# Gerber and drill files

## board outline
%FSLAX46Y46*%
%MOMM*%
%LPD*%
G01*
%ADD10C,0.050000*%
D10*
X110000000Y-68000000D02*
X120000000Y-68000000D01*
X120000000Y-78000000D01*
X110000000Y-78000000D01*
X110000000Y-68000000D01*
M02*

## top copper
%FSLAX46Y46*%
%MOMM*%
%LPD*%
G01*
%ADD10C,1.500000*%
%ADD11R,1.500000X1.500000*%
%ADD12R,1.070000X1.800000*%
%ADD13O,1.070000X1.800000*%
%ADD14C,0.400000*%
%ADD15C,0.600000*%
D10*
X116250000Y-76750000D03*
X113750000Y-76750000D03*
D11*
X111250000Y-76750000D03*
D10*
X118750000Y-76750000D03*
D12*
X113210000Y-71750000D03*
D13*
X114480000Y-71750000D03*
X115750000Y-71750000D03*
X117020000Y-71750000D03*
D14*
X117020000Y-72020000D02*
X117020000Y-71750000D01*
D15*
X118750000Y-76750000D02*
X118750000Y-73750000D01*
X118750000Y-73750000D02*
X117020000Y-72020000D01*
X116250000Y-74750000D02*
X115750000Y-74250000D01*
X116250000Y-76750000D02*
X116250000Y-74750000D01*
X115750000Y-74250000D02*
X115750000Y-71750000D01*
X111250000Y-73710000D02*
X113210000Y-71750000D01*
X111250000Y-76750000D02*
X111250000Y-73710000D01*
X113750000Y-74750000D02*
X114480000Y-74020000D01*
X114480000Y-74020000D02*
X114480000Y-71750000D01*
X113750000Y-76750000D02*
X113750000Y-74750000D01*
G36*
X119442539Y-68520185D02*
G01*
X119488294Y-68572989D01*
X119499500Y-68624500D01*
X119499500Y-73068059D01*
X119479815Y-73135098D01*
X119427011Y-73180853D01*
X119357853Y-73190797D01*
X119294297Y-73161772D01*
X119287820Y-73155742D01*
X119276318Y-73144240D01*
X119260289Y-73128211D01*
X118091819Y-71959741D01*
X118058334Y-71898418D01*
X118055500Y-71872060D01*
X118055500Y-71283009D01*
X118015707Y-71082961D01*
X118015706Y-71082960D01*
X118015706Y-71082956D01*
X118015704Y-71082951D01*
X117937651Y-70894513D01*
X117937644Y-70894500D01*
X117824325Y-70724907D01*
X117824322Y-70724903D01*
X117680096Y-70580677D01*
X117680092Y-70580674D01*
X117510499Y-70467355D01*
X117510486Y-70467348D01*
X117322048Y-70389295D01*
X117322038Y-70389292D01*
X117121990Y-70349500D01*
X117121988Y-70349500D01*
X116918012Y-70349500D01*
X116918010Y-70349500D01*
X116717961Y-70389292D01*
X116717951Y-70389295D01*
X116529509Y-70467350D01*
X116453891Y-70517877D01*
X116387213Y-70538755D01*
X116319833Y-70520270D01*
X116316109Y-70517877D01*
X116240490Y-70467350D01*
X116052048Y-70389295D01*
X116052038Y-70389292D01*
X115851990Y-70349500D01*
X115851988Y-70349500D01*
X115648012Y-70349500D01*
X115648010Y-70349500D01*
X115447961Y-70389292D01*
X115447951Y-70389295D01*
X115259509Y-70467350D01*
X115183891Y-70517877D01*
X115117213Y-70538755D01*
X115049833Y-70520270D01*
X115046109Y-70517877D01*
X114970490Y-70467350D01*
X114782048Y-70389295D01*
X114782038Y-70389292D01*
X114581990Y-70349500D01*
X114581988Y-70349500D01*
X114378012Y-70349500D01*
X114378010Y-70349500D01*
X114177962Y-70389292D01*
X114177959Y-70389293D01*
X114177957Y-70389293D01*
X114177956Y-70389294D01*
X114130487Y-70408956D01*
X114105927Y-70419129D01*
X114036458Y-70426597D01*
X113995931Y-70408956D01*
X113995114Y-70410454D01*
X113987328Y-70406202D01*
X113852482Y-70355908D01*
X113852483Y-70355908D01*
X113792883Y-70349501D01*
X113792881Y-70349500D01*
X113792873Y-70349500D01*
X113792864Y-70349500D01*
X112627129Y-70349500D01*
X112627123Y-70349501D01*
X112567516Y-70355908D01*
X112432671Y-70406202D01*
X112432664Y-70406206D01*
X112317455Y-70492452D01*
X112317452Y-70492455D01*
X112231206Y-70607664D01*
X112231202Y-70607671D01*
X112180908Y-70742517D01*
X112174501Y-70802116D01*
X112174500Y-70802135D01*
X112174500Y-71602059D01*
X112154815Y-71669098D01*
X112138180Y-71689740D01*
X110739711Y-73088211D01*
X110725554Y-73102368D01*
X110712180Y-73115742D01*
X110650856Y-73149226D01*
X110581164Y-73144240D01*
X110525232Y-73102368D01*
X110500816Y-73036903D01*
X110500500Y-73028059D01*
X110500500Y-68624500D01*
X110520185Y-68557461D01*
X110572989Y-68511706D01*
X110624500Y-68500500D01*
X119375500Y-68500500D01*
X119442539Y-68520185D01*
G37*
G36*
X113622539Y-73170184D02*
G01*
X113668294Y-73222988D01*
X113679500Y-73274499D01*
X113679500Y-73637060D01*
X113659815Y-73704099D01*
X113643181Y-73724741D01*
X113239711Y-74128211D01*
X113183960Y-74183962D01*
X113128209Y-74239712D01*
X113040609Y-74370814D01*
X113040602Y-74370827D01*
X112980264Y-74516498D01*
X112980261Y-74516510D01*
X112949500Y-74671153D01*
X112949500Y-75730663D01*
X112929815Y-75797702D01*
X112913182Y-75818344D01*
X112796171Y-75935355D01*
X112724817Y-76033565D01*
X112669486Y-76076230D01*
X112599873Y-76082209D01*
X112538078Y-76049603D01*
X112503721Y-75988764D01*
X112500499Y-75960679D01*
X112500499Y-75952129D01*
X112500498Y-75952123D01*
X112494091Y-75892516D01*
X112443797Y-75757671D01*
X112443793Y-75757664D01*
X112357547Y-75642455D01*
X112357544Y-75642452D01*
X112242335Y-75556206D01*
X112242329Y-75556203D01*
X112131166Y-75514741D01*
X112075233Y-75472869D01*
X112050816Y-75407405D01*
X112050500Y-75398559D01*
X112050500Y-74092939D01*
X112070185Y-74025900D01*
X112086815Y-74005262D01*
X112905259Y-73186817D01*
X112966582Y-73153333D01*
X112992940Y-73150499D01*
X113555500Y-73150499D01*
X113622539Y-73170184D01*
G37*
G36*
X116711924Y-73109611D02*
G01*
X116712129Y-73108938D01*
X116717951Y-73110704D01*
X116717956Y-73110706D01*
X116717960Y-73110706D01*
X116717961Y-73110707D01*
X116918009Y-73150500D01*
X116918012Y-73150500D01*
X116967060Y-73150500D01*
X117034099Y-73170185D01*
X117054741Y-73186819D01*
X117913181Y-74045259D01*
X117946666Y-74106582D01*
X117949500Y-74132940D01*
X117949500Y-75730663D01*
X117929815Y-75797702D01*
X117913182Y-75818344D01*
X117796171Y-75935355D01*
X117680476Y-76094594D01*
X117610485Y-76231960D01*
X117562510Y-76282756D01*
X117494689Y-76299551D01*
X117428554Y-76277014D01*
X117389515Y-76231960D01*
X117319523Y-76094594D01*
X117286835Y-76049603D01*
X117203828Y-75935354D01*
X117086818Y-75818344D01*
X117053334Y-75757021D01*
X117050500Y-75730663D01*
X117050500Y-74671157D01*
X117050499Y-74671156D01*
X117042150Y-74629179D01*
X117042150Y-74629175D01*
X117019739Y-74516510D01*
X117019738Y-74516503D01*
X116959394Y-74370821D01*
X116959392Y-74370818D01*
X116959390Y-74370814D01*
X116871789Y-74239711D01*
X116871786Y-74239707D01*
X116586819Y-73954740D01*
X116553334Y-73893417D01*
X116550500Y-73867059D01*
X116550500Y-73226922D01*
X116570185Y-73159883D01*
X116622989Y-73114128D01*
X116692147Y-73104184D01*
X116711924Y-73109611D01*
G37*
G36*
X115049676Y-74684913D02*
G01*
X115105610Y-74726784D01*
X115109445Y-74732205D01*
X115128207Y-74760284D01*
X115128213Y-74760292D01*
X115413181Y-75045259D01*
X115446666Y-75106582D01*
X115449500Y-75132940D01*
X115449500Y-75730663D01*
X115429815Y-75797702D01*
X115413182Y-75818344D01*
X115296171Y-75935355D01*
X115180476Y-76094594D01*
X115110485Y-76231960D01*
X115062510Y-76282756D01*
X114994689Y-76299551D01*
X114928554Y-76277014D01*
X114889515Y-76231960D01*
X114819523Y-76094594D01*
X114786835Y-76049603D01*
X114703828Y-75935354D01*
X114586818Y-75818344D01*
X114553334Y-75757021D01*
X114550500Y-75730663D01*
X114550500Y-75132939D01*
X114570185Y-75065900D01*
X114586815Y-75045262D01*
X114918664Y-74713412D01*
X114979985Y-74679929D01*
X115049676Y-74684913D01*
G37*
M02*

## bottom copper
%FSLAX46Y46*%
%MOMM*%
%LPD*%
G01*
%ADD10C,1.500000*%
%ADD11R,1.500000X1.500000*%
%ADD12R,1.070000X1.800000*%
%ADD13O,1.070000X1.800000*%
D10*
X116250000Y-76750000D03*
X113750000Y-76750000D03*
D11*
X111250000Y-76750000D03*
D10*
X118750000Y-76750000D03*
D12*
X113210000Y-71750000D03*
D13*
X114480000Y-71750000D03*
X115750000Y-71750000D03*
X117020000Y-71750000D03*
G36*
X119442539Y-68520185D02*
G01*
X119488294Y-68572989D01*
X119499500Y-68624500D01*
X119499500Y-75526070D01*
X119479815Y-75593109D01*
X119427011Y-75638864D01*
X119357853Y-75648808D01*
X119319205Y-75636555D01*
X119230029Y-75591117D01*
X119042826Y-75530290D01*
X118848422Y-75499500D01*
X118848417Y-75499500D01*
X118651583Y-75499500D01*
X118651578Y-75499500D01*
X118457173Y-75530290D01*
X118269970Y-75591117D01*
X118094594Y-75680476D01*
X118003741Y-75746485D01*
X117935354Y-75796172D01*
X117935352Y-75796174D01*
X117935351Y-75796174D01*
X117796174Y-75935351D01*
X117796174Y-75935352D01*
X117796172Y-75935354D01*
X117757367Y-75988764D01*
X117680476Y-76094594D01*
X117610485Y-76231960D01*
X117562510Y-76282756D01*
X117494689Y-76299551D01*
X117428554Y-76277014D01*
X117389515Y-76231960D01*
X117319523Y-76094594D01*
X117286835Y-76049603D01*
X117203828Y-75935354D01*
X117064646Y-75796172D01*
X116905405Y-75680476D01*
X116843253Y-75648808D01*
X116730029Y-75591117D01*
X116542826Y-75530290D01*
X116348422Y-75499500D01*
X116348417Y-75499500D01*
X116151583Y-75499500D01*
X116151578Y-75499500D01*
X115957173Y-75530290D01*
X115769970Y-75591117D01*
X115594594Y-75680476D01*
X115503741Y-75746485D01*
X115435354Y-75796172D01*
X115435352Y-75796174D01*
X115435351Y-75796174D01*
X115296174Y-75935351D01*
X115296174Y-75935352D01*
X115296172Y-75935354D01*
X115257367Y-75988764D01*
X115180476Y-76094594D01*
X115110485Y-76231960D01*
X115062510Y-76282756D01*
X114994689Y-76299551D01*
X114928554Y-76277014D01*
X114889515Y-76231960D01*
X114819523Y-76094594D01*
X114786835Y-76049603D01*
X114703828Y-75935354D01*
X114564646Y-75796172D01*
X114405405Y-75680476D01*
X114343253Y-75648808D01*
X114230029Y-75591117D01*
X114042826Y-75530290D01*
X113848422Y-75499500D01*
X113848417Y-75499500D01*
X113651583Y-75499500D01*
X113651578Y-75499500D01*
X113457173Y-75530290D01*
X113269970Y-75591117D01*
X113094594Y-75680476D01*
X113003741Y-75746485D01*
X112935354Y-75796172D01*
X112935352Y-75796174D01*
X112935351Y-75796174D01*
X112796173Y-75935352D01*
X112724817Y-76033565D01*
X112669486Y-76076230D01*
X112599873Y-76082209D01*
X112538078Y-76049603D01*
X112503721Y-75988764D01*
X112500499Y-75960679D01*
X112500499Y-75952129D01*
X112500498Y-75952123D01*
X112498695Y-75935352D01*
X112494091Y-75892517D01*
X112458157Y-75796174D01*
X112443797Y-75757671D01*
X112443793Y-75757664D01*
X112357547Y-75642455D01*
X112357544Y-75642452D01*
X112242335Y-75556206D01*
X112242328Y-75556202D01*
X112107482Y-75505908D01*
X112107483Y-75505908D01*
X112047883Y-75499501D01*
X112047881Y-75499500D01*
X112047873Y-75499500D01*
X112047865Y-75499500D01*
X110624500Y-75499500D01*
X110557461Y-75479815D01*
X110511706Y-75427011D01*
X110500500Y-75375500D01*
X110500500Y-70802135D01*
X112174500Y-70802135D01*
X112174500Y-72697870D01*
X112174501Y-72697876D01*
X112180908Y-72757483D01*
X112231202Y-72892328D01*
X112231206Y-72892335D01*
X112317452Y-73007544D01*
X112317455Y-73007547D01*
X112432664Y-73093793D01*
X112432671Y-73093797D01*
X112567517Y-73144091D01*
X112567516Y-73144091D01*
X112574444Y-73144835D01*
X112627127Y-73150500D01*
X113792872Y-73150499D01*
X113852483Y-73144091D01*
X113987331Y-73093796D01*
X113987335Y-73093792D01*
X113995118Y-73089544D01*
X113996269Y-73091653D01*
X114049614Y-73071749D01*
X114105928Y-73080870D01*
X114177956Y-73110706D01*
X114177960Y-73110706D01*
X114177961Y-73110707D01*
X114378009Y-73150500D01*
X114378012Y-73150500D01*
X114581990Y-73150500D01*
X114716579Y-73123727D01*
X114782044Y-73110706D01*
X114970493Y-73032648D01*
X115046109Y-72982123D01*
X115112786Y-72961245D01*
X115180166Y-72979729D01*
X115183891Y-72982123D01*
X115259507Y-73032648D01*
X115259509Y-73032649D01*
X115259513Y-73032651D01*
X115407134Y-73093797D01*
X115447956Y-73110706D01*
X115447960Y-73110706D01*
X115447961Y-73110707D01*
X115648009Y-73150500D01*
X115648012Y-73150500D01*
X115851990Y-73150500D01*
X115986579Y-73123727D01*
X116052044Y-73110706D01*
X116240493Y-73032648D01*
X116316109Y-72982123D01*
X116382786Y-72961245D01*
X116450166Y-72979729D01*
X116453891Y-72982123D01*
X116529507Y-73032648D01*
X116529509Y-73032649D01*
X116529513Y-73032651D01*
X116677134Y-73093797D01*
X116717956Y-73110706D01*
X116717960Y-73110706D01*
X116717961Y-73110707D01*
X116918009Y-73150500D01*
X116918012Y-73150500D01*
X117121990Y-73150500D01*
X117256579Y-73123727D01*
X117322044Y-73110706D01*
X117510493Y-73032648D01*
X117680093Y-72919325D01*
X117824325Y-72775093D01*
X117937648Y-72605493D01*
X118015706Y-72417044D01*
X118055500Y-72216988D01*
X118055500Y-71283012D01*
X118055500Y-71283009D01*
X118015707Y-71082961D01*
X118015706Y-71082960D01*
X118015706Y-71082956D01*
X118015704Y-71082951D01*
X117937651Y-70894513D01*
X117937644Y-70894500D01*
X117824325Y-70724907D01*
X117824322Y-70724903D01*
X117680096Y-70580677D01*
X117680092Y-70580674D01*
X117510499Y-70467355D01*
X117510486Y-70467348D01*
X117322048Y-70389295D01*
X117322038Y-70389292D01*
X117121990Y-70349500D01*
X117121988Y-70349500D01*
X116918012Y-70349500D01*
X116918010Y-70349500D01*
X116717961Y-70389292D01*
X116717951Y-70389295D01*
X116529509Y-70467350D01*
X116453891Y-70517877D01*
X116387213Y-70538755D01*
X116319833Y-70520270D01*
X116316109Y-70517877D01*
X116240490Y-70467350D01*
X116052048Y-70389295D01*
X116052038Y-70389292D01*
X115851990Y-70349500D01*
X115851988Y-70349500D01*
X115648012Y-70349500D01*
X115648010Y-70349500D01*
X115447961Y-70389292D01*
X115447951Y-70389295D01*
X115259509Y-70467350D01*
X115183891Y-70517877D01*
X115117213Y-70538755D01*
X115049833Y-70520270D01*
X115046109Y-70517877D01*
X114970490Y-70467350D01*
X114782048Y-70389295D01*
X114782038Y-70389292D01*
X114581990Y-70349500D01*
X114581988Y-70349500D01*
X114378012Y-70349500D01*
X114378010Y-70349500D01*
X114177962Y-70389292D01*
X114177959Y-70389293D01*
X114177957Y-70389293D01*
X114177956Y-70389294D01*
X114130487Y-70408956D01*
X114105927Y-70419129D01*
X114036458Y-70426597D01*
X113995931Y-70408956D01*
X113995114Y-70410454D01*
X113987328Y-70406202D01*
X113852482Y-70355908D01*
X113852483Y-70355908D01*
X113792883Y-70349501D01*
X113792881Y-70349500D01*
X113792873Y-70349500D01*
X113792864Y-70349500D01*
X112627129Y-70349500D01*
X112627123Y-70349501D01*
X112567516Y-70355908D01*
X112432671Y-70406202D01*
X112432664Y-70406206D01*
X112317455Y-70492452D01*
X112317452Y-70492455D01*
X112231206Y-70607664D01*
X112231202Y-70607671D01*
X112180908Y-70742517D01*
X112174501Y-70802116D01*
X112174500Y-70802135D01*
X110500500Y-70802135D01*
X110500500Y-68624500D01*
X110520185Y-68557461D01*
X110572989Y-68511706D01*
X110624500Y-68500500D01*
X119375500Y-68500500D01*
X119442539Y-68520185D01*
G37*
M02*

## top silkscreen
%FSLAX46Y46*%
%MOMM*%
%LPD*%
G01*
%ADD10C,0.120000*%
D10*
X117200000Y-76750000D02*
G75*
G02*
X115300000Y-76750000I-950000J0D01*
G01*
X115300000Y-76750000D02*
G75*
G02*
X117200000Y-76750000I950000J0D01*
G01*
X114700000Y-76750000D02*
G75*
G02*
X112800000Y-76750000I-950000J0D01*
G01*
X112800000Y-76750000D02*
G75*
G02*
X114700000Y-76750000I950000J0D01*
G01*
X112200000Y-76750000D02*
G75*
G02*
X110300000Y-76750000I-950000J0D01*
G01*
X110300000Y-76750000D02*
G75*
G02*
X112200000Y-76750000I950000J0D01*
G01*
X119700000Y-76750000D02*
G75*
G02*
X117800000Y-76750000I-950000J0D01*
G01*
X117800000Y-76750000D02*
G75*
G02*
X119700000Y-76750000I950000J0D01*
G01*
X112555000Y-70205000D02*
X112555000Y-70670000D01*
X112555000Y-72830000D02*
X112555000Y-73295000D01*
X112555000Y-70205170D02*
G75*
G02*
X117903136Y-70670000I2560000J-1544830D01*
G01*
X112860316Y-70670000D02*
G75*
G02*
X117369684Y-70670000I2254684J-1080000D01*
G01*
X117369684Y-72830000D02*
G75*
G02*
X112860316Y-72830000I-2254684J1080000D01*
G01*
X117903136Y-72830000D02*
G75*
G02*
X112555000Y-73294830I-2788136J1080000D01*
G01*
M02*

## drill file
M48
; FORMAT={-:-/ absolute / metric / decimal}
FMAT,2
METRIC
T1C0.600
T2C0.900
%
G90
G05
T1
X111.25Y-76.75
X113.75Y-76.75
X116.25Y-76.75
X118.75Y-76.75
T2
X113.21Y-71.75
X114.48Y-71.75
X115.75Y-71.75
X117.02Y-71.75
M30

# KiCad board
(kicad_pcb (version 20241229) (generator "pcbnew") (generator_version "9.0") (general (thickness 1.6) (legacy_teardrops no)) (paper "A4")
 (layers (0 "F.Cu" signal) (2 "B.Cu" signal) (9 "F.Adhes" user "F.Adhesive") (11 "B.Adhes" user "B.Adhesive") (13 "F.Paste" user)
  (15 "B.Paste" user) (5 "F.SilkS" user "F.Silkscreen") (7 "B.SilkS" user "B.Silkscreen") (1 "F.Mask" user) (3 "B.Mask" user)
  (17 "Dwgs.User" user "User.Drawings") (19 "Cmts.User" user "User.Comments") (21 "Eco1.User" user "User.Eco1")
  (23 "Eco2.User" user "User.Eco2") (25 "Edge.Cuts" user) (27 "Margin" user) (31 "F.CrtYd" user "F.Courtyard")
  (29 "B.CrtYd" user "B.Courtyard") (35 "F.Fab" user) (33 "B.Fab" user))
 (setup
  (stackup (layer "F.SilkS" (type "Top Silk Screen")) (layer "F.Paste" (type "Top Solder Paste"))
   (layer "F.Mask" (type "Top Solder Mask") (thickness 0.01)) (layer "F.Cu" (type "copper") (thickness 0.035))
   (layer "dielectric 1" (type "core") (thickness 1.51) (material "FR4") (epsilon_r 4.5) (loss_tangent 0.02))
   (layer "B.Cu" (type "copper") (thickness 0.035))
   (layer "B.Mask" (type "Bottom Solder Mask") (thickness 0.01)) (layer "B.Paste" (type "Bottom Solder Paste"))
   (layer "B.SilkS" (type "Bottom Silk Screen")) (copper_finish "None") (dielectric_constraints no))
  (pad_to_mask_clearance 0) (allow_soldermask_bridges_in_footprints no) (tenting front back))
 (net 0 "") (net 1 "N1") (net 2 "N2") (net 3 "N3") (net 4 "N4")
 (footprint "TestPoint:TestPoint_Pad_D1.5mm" (layer "F.Cu") (at 116.25 76.75)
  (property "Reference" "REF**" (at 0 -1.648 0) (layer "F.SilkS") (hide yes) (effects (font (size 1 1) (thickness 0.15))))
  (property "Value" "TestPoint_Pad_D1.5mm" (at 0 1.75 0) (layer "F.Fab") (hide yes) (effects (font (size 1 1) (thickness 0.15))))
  (fp_circle (center 0 0) (end 0 0.95) (stroke (width 0.12) (type solid)) (fill no) (layer "F.SilkS"))
  (pad "1" thru_hole circle (at 0 0) (size 1.5 1.5) (drill 0.6) (layers "*.Cu" "*.Mask") (remove_unused_layers no) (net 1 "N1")))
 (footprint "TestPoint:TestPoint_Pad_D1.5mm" (layer "F.Cu") (at 113.75 76.75)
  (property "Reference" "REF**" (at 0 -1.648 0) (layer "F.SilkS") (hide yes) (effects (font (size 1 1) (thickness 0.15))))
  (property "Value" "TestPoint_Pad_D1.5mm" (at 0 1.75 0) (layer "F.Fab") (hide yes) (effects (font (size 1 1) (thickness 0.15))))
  (fp_circle (center 0 0) (end 0 0.95) (stroke (width 0.12) (type solid)) (fill no) (layer "F.SilkS"))
  (pad "1" thru_hole circle (at 0 0) (size 1.5 1.5) (drill 0.6) (layers "*.Cu" "*.Mask") (remove_unused_layers no) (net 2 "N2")))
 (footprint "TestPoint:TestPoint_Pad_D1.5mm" (layer "F.Cu") (at 111.25 76.75)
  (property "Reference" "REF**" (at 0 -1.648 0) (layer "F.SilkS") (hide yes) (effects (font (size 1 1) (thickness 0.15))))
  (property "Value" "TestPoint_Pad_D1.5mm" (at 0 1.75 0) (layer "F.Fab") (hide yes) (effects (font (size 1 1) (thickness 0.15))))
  (fp_circle (center 0 0) (end 0 0.95) (stroke (width 0.12) (type solid)) (fill no) (layer "F.SilkS"))
  (pad "1" thru_hole rect (at 0 0) (size 1.5 1.5) (drill 0.6) (layers "*.Cu" "*.Mask") (remove_unused_layers no) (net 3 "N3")))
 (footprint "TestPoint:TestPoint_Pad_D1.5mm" (layer "F.Cu") (at 118.75 76.75)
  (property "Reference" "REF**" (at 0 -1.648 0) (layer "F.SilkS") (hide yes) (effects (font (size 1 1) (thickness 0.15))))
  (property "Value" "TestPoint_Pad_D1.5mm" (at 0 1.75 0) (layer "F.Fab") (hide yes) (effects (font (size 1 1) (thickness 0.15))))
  (fp_circle (center 0 0) (end 0 0.95) (stroke (width 0.12) (type solid)) (fill no) (layer "F.SilkS"))
  (pad "1" thru_hole circle (at 0 0) (size 1.5 1.5) (drill 0.6) (layers "*.Cu" "*.Mask") (remove_unused_layers no) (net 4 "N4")))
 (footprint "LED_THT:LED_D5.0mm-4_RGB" (layer "F.Cu") (at 113.21 71.75)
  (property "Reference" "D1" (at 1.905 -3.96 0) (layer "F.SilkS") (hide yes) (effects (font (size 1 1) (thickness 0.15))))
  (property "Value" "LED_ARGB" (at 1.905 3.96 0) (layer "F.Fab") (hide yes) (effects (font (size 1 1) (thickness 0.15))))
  (fp_line (start -0.655 -1.545) (end -0.655 -1.08) (stroke (width 0.12) (type solid)) (layer "F.SilkS"))
  (fp_line (start -0.655 1.08) (end -0.655 1.545) (stroke (width 0.12) (type solid)) (layer "F.SilkS"))
  (fp_arc (start -0.655 -1.54483) (mid 2.163898 -2.97877) (end 4.693136 -1.08) (stroke (width 0.12) (type solid)) (layer "F.SilkS"))
  (fp_arc (start -0.349684 -1.08) (mid 1.905 -2.5) (end 4.159684 -1.08) (stroke (width 0.12) (type solid)) (layer "F.SilkS"))
  (fp_arc (start 4.159684 1.08) (mid 1.905 2.5) (end -0.349684 1.08) (stroke (width 0.12) (type solid)) (layer "F.SilkS"))
  (fp_arc (start 4.693136 1.08) (mid 2.163898 2.97877) (end -0.655 1.54483) (stroke (width 0.12) (type solid)) (layer "F.SilkS"))
  (pad "1" thru_hole rect (at 0 0) (size 1.07 1.8) (drill 0.9) (layers "*.Cu" "*.Mask") (remove_unused_layers no) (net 3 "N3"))
  (pad "2" thru_hole oval (at 1.27 0) (size 1.07 1.8) (drill 0.9) (layers "*.Cu" "*.Mask") (remove_unused_layers no) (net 2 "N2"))
  (pad "3" thru_hole oval (at 2.54 0) (size 1.07 1.8) (drill 0.9) (layers "*.Cu" "*.Mask") (remove_unused_layers no) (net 1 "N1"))
  (pad "4" thru_hole oval (at 3.81 0) (size 1.07 1.8) (drill 0.9) (layers "*.Cu" "*.Mask") (remove_unused_layers no) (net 4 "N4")))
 (gr_rect (start 110 68) (end 120 78) (stroke (width 0.05) (type default)) (fill no) (layer "Edge.Cuts"))
 (segment (start 117.02 72.02) (end 117.02 71.75) (width 0.4) (layer "F.Cu") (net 4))
 (segment (start 118.75 76.75) (end 118.75 73.75) (width 0.6) (layer "F.Cu") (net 4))
 (segment (start 118.75 73.75) (end 117.02 72.02) (width 0.6) (layer "F.Cu") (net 4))
 (segment (start 116.25 74.75) (end 115.75 74.25) (width 0.6) (layer "F.Cu") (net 1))
 (segment (start 116.25 76.75) (end 116.25 74.75) (width 0.6) (layer "F.Cu") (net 1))
 (segment (start 115.75 74.25) (end 115.75 71.75) (width 0.6) (layer "F.Cu") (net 1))
 (segment (start 111.25 73.71) (end 113.21 71.75) (width 0.6) (layer "F.Cu") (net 3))
 (segment (start 111.25 76.75) (end 111.25 73.71) (width 0.6) (layer "F.Cu") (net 3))
 (segment (start 113.75 74.75) (end 114.48 74.02) (width 0.6) (layer "F.Cu") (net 2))
 (segment (start 114.48 74.02) (end 114.48 71.75) (width 0.6) (layer "F.Cu") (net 2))
 (segment (start 113.75 76.75) (end 113.75 74.75) (width 0.6) (layer "F.Cu") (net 2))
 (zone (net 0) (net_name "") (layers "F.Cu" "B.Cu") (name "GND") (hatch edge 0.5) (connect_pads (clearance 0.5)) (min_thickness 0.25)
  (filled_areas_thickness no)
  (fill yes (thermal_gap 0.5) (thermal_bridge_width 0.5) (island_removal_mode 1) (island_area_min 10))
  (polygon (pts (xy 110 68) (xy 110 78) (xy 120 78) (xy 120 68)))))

